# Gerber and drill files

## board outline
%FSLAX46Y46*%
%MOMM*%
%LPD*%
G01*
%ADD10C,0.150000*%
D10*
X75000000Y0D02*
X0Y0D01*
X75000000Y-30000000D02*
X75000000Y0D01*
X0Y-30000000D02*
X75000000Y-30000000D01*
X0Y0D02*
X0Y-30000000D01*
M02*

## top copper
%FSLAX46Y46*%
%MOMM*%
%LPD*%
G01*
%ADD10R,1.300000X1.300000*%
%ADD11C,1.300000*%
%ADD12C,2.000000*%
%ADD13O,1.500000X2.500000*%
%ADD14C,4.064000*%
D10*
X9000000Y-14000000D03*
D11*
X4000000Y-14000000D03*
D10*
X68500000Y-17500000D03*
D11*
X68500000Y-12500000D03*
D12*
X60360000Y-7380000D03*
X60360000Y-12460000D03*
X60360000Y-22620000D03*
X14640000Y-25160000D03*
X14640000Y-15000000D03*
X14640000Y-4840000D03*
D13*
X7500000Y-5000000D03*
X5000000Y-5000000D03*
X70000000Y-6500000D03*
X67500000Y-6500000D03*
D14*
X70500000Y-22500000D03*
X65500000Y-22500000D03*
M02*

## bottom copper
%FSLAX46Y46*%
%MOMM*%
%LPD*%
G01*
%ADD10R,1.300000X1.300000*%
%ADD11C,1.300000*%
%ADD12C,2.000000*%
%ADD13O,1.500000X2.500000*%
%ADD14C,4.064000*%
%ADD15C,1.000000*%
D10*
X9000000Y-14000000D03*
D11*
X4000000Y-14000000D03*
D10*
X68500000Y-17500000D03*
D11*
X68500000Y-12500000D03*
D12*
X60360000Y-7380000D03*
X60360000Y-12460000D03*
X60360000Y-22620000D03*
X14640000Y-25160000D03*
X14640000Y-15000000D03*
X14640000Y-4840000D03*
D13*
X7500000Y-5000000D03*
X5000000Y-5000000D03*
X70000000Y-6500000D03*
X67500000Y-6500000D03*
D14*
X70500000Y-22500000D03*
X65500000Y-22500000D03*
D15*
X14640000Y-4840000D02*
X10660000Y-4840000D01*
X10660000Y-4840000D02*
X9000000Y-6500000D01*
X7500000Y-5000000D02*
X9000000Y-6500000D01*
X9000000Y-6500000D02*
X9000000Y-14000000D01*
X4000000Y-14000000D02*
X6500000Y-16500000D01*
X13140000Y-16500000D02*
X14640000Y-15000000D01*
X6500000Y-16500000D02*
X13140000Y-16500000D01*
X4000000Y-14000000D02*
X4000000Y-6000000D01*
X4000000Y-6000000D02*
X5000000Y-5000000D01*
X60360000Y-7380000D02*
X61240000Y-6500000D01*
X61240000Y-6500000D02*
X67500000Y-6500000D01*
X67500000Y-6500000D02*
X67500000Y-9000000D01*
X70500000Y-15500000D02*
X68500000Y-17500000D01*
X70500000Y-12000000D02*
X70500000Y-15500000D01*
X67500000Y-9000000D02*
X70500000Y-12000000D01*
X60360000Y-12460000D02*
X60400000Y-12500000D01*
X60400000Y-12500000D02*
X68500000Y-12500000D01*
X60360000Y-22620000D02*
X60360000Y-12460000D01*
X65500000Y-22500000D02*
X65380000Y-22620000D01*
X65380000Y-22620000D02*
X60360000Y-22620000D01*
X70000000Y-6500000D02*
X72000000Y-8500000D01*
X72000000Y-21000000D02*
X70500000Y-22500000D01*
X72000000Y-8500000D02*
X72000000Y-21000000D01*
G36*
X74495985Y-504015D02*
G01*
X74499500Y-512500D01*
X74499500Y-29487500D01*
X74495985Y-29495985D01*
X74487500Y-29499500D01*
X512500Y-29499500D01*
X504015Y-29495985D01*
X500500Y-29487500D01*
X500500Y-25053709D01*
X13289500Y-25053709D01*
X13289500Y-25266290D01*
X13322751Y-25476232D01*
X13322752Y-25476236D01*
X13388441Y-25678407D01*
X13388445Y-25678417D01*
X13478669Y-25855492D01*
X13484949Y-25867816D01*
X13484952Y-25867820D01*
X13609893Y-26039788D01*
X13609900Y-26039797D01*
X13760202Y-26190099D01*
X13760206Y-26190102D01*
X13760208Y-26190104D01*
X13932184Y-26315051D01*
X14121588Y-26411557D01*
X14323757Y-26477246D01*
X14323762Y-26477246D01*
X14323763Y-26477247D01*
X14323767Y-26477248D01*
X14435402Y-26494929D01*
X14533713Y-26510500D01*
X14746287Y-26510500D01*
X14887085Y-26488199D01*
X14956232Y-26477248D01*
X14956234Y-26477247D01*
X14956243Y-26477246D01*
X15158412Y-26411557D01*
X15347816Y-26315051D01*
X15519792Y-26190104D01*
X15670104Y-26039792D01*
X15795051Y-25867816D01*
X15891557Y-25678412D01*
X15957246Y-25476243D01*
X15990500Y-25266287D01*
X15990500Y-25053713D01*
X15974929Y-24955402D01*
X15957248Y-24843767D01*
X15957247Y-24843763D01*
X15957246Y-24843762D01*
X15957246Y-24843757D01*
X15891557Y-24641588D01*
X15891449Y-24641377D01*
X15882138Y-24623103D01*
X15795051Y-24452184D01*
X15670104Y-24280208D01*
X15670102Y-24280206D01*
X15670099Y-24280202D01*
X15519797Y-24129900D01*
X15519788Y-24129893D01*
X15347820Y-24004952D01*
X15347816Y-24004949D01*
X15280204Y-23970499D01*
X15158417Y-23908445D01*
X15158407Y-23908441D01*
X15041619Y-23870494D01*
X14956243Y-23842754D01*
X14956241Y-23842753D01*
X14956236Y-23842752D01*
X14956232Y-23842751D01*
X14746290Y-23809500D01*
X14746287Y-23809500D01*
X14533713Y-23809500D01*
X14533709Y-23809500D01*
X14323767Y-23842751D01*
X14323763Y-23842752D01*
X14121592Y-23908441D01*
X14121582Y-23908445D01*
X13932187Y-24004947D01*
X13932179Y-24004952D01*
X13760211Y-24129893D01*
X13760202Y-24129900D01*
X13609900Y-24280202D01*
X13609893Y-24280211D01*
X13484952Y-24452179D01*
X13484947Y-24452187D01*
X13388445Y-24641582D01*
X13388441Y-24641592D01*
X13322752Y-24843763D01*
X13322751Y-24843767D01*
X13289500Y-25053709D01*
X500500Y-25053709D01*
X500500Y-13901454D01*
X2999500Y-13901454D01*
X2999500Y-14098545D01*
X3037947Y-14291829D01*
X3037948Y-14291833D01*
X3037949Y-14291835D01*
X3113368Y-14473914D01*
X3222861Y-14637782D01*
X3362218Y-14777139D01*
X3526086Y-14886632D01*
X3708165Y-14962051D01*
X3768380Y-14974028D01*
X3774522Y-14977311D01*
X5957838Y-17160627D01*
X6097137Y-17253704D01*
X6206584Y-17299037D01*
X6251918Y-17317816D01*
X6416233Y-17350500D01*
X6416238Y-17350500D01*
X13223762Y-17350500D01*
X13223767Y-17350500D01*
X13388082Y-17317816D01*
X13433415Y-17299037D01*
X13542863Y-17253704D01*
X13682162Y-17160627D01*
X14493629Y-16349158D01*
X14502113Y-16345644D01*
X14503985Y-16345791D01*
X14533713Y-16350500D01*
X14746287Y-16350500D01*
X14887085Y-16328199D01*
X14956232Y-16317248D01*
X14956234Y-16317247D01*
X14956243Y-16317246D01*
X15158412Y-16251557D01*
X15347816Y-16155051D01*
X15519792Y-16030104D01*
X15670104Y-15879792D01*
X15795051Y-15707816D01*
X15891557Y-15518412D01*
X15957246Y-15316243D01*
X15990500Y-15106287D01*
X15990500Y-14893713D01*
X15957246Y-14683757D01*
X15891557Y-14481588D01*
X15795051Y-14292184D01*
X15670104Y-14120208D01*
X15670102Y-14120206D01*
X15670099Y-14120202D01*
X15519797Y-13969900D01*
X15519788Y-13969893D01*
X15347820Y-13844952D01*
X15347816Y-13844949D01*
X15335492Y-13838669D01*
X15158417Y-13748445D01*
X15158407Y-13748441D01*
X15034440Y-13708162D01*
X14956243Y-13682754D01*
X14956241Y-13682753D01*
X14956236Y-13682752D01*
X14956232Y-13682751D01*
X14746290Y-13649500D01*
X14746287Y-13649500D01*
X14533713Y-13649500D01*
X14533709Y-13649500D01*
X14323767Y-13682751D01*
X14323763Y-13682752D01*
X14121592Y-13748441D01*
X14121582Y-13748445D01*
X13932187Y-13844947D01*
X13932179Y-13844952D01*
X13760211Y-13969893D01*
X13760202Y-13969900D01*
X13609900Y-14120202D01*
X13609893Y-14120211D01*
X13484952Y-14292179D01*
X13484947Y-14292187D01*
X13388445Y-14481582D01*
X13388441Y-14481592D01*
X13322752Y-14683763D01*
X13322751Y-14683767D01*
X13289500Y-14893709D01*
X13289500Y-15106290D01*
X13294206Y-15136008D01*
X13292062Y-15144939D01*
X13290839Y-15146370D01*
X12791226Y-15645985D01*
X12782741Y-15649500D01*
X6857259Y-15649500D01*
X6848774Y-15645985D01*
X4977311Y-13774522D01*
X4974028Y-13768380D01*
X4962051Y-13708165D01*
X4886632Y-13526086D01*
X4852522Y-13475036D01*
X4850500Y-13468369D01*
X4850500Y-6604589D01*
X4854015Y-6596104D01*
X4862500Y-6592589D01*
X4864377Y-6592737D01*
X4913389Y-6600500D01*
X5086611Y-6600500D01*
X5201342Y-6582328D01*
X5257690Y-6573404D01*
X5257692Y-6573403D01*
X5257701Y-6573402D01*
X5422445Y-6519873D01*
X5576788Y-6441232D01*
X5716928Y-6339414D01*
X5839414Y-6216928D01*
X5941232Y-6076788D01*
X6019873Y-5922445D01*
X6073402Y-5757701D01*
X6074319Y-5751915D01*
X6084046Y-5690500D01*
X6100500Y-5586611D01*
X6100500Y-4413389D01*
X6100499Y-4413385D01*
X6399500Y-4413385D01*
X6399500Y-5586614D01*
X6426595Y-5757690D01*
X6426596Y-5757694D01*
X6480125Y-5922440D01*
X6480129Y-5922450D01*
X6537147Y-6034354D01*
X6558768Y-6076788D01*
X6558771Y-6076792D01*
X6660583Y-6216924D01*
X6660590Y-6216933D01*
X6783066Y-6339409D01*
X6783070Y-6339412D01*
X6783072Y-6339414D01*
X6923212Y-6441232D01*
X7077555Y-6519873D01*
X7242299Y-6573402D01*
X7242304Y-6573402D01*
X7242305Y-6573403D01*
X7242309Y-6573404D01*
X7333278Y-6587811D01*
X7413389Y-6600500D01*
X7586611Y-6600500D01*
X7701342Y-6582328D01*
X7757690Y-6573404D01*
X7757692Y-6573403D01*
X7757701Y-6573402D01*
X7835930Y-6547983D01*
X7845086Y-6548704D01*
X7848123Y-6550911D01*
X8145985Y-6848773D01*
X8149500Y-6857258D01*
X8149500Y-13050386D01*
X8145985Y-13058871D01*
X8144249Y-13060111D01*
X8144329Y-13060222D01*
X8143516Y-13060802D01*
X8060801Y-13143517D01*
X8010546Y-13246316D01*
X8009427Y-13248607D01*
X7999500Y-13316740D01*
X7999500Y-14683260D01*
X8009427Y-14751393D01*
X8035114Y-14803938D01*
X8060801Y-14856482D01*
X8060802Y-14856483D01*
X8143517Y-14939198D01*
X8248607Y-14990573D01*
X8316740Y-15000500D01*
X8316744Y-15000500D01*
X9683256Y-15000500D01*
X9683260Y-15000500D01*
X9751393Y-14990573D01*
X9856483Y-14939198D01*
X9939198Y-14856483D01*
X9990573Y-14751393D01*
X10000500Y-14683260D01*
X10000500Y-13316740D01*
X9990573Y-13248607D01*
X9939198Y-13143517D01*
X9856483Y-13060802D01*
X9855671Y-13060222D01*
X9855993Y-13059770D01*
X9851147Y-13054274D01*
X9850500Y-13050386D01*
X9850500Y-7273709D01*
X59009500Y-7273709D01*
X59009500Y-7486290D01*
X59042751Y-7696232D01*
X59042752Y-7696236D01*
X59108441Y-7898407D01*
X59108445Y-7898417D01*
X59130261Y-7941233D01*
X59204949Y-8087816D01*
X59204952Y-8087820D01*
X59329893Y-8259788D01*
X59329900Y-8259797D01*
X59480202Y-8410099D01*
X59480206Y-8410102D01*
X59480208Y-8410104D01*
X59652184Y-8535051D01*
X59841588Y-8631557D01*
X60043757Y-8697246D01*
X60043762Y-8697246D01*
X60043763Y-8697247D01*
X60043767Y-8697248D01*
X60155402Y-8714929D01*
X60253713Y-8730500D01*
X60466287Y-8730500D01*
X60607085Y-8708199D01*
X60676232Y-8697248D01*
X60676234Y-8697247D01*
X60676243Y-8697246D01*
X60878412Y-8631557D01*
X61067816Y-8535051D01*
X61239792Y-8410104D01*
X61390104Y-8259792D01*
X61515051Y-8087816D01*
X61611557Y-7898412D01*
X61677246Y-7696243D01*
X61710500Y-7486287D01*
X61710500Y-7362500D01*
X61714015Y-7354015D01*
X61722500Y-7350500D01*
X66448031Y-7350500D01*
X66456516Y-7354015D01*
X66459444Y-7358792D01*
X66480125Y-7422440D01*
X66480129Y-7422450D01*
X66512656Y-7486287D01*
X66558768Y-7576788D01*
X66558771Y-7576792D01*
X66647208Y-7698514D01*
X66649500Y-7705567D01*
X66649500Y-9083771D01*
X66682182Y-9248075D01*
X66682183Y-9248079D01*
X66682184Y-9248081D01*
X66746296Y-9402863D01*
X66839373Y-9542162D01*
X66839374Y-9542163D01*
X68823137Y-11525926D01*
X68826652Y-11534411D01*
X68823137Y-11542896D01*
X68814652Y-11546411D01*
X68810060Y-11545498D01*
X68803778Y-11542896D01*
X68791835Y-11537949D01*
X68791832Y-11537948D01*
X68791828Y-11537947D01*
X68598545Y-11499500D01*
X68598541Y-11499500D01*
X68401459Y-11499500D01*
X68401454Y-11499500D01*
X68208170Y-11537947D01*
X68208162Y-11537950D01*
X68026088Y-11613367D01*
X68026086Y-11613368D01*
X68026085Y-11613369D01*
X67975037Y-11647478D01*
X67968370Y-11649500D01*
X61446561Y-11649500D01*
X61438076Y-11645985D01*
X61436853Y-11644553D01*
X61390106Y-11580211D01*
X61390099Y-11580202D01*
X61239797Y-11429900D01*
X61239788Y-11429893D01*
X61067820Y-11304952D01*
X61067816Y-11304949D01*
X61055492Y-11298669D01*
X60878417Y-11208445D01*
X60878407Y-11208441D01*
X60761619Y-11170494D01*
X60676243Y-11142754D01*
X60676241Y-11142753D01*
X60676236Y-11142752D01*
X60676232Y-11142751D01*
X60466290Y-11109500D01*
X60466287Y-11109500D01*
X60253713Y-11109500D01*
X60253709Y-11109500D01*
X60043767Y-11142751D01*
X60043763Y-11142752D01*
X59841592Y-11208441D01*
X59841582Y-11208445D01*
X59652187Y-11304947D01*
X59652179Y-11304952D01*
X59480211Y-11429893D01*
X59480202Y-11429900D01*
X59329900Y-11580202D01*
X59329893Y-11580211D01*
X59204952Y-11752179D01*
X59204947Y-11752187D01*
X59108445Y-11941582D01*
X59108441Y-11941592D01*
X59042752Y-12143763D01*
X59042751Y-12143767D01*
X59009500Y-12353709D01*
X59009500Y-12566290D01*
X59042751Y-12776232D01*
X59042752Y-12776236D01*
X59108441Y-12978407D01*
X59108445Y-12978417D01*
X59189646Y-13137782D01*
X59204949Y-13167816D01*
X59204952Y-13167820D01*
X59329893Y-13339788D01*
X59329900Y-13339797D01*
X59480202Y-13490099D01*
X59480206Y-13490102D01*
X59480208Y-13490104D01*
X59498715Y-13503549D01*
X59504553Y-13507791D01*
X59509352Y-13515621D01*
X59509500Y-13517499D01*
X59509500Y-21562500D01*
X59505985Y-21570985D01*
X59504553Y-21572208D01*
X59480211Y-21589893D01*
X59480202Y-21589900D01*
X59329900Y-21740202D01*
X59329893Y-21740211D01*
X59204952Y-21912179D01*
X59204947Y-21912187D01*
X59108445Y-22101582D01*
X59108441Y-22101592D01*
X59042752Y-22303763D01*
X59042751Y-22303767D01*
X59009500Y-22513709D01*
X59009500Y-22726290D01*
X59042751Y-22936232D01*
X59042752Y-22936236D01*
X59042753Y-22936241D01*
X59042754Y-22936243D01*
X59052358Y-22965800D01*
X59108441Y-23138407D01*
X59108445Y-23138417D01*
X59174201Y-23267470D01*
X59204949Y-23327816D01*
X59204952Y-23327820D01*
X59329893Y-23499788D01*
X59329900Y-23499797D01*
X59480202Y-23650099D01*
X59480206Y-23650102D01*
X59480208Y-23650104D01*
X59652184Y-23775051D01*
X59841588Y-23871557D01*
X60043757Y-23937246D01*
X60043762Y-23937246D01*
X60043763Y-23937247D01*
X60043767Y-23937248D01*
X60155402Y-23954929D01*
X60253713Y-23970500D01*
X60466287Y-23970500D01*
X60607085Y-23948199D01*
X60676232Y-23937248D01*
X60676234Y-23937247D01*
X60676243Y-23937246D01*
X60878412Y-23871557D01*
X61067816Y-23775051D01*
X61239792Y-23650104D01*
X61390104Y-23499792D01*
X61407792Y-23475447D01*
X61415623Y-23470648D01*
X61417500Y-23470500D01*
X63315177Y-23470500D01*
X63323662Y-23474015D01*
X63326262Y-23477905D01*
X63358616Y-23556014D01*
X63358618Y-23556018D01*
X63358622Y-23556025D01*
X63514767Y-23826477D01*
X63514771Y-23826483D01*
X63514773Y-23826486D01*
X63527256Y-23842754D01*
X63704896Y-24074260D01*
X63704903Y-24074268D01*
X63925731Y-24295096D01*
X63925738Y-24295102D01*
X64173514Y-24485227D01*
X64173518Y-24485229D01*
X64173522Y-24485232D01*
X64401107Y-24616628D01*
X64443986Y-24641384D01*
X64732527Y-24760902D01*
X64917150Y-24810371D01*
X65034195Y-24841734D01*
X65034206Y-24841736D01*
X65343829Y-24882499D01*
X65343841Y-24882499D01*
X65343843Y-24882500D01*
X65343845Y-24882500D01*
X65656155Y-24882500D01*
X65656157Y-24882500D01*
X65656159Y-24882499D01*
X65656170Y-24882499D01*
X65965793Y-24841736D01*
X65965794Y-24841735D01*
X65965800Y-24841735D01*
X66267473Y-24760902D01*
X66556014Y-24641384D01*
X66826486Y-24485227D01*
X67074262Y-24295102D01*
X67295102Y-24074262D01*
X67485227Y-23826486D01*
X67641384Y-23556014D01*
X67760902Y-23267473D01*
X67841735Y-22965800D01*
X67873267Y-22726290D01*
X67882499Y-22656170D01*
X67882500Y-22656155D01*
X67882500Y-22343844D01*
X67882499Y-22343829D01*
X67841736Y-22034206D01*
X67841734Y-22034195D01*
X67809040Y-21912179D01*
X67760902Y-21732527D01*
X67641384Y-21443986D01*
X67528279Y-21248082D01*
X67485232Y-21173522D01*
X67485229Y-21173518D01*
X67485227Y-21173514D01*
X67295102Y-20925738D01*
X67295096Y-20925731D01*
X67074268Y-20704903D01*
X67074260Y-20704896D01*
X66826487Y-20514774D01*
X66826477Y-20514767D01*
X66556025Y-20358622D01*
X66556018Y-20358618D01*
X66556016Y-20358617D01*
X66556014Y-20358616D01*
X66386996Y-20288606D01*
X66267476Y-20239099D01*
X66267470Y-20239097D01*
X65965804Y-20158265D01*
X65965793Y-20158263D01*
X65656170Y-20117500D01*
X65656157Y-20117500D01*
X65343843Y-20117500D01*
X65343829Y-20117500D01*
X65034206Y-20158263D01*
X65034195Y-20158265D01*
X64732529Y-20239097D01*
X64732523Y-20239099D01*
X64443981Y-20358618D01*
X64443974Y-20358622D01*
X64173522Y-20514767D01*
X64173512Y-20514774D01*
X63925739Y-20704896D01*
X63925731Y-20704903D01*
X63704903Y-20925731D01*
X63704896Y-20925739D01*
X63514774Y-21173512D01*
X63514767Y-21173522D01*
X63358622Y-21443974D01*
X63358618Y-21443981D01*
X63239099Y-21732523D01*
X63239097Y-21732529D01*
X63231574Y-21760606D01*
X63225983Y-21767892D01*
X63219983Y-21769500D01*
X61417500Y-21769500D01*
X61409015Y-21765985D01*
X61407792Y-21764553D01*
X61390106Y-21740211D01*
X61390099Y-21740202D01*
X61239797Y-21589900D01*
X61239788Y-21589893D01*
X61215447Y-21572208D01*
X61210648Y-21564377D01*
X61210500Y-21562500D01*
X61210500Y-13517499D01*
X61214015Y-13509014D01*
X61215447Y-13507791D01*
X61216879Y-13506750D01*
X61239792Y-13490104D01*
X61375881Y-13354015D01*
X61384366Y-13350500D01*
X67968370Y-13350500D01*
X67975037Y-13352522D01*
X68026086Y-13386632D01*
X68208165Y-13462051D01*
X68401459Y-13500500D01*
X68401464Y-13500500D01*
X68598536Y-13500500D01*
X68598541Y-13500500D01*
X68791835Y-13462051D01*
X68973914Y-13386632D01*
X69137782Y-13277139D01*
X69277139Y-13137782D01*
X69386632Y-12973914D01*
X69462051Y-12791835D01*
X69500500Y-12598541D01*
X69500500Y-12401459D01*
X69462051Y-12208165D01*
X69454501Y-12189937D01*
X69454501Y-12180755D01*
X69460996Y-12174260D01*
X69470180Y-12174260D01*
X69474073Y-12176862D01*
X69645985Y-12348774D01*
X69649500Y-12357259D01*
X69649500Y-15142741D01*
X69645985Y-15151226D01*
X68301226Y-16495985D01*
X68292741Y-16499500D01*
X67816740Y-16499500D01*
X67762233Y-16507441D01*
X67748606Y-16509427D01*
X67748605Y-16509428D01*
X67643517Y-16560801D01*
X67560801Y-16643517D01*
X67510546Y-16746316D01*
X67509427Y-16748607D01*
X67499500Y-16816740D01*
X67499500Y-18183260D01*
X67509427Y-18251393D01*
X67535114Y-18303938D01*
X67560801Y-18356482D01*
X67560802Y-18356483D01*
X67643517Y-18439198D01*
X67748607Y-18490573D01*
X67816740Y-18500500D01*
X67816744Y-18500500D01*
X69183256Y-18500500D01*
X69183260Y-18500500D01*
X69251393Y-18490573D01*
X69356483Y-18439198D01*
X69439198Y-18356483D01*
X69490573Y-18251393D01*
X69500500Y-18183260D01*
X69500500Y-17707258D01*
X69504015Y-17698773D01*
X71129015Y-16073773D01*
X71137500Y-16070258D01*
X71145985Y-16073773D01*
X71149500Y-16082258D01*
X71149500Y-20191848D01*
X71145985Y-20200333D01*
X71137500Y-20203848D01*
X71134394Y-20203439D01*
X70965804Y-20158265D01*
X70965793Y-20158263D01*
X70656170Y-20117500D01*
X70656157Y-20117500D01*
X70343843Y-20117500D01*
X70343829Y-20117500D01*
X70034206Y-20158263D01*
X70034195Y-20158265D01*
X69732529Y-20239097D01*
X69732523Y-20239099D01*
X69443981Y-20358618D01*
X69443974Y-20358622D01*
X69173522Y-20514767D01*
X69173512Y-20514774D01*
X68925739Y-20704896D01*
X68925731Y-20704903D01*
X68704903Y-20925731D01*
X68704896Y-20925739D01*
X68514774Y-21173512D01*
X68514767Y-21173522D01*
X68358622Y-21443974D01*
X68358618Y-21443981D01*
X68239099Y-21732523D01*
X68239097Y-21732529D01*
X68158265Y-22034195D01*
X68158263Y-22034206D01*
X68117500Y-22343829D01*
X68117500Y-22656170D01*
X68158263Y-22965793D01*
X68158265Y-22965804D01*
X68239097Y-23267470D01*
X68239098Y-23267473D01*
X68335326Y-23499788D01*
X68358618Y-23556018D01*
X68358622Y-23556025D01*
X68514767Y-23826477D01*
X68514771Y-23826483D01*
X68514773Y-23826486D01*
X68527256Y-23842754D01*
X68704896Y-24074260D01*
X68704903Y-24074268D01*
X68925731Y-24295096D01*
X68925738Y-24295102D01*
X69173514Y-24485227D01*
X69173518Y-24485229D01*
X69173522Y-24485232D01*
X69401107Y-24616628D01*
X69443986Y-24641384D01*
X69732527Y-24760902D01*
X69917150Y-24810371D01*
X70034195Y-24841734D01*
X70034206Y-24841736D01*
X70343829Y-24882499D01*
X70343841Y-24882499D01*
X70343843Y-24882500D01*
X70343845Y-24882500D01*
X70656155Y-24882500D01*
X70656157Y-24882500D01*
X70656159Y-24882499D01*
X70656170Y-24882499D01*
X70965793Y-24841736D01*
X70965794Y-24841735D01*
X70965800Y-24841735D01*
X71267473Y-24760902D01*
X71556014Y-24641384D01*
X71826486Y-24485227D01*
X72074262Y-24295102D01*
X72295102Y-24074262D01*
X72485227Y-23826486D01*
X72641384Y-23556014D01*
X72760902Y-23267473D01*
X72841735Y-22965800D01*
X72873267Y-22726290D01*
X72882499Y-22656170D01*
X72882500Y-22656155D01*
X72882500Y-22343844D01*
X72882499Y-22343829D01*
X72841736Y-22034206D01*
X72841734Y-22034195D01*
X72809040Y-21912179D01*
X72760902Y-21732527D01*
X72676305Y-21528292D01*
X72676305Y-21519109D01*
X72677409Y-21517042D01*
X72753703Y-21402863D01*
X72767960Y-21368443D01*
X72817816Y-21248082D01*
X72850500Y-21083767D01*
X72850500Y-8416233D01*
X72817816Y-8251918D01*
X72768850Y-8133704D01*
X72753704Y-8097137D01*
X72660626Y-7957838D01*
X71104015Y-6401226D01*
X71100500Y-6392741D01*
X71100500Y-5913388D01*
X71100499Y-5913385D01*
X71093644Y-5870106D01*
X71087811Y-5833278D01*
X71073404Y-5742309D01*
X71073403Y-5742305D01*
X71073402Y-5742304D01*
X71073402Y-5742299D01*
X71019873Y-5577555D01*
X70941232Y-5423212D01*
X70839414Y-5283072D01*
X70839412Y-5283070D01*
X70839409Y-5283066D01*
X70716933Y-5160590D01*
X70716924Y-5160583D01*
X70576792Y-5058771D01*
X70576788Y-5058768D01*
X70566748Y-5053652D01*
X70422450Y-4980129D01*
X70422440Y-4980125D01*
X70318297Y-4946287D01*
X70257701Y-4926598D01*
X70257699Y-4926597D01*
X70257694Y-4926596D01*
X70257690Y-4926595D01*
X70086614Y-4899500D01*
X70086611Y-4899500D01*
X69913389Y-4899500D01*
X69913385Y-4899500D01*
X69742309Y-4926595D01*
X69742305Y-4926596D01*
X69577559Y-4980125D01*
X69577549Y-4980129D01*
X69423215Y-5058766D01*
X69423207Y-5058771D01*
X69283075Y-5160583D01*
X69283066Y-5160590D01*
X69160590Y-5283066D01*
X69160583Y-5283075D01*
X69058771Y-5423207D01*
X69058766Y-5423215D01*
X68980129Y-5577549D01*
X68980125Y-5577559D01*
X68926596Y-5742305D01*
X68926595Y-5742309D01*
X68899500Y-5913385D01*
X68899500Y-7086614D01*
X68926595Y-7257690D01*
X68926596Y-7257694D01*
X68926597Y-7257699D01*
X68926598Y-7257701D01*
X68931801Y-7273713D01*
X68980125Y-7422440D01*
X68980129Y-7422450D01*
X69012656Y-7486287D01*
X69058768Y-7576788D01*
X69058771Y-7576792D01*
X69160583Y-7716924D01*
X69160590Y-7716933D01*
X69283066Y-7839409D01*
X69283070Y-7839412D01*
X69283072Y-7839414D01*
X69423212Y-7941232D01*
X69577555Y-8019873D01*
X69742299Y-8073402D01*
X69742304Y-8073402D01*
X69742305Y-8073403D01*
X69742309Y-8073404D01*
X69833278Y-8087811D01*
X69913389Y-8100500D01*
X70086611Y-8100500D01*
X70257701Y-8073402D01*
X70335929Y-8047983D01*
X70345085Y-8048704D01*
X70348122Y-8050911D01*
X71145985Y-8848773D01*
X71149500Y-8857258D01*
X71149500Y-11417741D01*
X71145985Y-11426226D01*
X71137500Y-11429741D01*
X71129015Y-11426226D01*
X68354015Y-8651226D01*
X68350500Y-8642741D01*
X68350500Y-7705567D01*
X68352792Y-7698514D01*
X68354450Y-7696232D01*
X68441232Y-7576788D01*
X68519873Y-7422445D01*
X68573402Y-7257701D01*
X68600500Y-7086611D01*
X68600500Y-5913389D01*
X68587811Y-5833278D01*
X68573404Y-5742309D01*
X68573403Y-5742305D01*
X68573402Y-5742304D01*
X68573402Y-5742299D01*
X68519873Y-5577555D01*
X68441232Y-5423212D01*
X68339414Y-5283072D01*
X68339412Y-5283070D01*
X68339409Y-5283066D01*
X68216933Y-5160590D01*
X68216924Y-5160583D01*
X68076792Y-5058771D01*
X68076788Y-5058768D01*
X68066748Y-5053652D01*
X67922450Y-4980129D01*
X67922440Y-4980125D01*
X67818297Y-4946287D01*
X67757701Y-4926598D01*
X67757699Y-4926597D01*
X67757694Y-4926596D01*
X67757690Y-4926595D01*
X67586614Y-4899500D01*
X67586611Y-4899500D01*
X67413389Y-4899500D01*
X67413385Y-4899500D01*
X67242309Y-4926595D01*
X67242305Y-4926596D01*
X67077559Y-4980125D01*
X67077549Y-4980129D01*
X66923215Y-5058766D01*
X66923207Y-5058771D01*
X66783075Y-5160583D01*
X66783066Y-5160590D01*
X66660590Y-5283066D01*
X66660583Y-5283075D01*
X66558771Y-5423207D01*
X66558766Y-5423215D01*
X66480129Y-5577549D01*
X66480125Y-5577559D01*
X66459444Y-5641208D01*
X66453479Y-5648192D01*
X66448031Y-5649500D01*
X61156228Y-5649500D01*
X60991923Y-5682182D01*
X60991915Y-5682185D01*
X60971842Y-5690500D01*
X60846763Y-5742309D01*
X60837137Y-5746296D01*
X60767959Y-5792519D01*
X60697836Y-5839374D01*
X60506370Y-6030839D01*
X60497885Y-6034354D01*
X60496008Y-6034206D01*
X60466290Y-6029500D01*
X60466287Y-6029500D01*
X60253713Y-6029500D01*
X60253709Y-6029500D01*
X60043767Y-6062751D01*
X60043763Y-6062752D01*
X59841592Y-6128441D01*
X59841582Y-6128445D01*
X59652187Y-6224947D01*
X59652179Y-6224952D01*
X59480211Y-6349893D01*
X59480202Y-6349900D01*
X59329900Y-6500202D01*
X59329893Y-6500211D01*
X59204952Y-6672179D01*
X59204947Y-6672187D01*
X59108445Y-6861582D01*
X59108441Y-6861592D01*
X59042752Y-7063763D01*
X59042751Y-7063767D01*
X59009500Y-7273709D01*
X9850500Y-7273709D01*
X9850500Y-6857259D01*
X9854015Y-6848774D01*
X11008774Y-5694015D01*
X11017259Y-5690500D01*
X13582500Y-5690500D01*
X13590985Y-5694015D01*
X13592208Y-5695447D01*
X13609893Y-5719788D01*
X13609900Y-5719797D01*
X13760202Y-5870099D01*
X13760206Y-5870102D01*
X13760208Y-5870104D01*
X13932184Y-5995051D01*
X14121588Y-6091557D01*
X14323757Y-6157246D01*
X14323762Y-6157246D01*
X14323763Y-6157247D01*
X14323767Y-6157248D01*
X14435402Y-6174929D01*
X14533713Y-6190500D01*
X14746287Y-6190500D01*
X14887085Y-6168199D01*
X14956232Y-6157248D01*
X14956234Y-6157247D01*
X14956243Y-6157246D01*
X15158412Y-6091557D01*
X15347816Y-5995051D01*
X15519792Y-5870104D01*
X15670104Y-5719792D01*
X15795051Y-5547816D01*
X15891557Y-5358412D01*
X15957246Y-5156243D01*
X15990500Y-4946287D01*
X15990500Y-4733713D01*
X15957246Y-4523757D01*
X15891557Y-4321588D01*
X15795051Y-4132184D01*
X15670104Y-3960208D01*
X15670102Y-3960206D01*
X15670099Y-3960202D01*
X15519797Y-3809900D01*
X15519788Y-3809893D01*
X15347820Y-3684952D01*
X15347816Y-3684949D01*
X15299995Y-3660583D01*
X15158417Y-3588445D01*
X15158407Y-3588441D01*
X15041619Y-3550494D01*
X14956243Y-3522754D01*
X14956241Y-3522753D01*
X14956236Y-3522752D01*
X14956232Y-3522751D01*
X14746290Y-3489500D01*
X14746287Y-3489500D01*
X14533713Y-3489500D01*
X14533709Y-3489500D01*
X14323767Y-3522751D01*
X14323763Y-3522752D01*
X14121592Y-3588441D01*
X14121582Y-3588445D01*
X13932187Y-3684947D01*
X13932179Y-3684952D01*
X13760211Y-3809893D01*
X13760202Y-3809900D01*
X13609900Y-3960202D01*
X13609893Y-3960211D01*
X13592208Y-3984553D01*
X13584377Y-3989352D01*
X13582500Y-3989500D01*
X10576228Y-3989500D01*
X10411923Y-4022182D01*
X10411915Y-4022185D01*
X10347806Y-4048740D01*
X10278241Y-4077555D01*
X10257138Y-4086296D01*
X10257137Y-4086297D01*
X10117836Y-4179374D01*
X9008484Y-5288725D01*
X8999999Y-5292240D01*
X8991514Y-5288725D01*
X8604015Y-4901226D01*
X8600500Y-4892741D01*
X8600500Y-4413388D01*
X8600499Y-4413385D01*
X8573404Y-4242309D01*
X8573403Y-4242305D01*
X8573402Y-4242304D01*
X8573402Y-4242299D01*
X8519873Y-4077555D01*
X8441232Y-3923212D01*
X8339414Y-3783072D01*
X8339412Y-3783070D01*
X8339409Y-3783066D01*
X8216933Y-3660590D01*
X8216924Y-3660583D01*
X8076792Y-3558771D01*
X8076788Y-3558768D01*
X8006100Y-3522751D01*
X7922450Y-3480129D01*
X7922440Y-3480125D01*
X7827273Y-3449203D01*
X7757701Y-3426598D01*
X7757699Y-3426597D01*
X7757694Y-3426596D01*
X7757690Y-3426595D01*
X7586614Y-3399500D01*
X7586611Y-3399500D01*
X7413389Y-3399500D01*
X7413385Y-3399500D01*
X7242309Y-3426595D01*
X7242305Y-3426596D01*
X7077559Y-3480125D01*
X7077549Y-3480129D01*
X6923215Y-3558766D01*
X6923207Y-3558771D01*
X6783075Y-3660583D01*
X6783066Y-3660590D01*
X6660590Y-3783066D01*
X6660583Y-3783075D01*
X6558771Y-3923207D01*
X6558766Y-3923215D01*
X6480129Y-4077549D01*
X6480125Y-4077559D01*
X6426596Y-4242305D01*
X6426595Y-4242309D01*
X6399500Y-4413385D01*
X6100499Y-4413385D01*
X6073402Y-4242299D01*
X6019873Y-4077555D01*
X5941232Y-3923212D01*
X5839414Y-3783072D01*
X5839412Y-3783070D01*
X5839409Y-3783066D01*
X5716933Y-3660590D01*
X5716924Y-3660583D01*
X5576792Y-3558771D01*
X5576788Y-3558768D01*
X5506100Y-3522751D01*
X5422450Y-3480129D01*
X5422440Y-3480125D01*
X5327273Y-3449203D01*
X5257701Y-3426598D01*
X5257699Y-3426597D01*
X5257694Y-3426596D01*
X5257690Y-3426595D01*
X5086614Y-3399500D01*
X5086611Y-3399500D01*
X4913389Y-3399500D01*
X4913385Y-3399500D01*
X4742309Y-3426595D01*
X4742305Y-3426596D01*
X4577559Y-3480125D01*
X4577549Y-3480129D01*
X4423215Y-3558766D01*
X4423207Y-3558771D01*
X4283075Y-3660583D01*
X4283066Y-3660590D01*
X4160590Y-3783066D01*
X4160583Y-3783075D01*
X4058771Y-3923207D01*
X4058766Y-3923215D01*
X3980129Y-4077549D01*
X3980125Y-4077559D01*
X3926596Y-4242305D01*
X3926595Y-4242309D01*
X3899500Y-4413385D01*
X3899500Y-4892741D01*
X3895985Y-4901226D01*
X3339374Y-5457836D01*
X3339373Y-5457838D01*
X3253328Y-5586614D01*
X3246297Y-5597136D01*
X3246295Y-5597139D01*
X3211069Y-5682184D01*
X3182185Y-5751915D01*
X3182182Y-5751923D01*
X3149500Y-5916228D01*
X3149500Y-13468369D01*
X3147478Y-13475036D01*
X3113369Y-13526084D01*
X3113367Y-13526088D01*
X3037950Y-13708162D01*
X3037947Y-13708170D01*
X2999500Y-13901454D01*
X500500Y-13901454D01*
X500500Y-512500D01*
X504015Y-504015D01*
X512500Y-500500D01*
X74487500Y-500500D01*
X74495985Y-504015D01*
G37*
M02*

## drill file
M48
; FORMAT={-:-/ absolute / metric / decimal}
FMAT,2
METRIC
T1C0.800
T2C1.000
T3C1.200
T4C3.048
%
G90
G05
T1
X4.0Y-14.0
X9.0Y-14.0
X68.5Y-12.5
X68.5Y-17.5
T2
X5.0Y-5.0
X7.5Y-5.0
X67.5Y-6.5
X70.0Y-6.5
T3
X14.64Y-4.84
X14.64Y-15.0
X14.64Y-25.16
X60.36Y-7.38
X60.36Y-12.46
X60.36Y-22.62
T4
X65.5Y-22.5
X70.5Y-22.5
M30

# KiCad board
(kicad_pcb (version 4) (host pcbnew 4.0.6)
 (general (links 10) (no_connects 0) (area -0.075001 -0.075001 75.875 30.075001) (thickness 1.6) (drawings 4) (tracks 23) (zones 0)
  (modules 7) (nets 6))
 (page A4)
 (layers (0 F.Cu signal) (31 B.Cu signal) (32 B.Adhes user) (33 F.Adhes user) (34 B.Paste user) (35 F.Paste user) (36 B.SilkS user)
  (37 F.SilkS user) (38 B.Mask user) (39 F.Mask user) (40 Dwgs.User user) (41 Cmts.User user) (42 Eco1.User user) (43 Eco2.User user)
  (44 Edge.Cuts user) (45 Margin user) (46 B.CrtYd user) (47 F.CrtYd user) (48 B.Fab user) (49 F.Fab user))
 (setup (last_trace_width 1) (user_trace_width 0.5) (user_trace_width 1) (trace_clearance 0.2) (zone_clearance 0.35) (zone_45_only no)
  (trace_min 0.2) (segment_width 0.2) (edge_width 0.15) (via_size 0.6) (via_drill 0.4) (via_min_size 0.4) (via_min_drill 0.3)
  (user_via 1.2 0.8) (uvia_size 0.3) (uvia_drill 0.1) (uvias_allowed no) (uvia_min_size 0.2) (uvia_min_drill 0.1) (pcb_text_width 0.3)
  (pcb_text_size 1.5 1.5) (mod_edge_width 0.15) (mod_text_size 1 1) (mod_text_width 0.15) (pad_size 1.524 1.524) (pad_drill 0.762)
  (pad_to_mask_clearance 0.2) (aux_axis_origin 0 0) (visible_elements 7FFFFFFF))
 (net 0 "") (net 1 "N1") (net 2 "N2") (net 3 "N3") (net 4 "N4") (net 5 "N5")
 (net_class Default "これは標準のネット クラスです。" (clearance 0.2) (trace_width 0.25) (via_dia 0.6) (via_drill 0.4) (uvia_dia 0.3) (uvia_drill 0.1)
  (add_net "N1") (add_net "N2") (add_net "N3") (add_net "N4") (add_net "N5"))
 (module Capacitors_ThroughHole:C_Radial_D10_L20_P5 (layer F.Cu) (at 9 14 180)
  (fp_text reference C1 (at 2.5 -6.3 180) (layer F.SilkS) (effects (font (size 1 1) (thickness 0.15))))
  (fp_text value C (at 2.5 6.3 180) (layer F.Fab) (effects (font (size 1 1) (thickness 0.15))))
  (pad 1 thru_hole rect (at 0 0 180) (size 1.3 1.3) (drill 0.8) (layers *.Cu *.Mask F.SilkS) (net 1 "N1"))
  (pad 2 thru_hole circle (at 5 0 180) (size 1.3 1.3) (drill 0.8) (layers *.Cu *.Mask F.SilkS) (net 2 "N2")))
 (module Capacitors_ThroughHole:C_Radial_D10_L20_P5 (layer F.Cu) (at 68.5 17.5 90)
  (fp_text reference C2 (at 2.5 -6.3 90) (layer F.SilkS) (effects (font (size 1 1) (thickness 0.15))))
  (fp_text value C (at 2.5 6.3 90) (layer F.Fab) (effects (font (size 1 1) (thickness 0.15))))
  (pad 1 thru_hole rect (at 0 0 90) (size 1.3 1.3) (drill 0.8) (layers *.Cu *.Mask F.SilkS) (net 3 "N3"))
  (pad 2 thru_hole circle (at 5 0 90) (size 1.3 1.3) (drill 0.8) (layers *.Cu *.Mask F.SilkS) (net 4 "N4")))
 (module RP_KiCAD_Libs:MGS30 (layer F.Cu) (at 37.5 15)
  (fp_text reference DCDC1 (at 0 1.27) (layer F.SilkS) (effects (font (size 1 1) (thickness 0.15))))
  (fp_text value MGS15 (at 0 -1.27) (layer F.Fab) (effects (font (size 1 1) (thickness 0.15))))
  (pad 6 thru_hole circle (at 22.86 -7.62) (size 2 2) (drill 1.2) (layers *.Cu *.Mask) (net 3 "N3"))
  (pad 5 thru_hole circle (at 22.86 -2.54) (size 2 2) (drill 1.2) (layers *.Cu *.Mask) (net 4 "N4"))
  (pad 4 thru_hole circle (at 22.86 7.62) (size 2 2) (drill 1.2) (layers *.Cu *.Mask) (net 4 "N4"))
  (pad 2 thru_hole circle (at -22.86 10.16) (size 2 2) (drill 1.2) (layers *.Cu *.Mask))
  (pad 3 thru_hole circle (at -22.86 0) (size 2 2) (drill 1.2) (layers *.Cu *.Mask) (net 2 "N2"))
  (pad 1 thru_hole circle (at -22.86 -10.16) (size 2 2) (drill 1.2) (layers *.Cu *.Mask) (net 1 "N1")))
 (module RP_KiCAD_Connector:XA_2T (layer F.Cu) (at 7.5 5 180)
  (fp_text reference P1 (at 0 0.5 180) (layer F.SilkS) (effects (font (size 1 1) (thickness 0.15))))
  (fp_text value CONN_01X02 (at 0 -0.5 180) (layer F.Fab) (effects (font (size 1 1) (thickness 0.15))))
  (pad 2 thru_hole oval (at 0 0 180) (size 1.5 2.5) (drill 1) (layers *.Cu *.Mask F.SilkS) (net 1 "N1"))
  (pad 1 thru_hole oval (at 2.5 0 180) (size 1.5 2.5) (drill 1) (layers *.Cu *.Mask F.SilkS) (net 2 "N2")))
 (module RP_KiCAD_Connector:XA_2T (layer F.Cu) (at 70 6.5 180)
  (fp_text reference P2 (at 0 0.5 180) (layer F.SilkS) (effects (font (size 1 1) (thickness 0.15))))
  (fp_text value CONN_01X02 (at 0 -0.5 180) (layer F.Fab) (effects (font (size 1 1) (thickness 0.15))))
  (pad 2 thru_hole oval (at 0 0 180) (size 1.5 2.5) (drill 1) (layers *.Cu *.Mask F.SilkS) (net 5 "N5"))
  (pad 1 thru_hole oval (at 2.5 0 180) (size 1.5 2.5) (drill 1) (layers *.Cu *.Mask F.SilkS) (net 3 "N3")))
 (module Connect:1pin (layer F.Cu) (at 70.5 22.5)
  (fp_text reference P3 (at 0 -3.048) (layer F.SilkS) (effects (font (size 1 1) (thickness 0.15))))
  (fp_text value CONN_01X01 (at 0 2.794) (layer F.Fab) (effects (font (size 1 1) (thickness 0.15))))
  (pad 1 thru_hole circle (at 0 0) (size 4.064 4.064) (drill 3.048) (layers *.Cu *.Mask F.SilkS) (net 5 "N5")))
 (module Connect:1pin (layer F.Cu) (at 65.5 22.5)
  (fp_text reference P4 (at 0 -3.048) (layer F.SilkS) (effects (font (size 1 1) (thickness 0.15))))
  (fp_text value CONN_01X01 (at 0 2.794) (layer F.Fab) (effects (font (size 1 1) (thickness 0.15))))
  (pad 1 thru_hole circle (at 0 0) (size 4.064 4.064) (drill 3.048) (layers *.Cu *.Mask F.SilkS) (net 4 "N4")))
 (gr_line (start 75 0) (end 0 0) (angle 90) (layer Edge.Cuts) (width 0.15))
 (gr_line (start 75 30) (end 75 0) (angle 90) (layer Edge.Cuts) (width 0.15))
 (gr_line (start 0 30) (end 75 30) (angle 90) (layer Edge.Cuts) (width 0.15))
 (gr_line (start 0 0) (end 0 30) (angle 90) (layer Edge.Cuts) (width 0.15))
 (segment (start 14.64 4.84) (end 10.66 4.84) (width 1) (layer B.Cu) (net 1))
 (segment (start 10.66 4.84) (end 9 6.5) (width 1) (layer B.Cu) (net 1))
 (segment (start 7.5 5) (end 9 6.5) (width 1) (layer B.Cu) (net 1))
 (segment (start 9 6.5) (end 9 14) (width 1) (layer B.Cu) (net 1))
 (segment (start 4 14) (end 6.5 16.5) (width 1) (layer B.Cu) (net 2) (status 400000))
 (segment (start 13.14 16.5) (end 14.64 15) (width 1) (layer B.Cu) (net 2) (status 800000))
 (segment (start 6.5 16.5) (end 13.14 16.5) (width 1) (layer B.Cu) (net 2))
 (segment (start 4 14) (end 4 6) (width 1) (layer B.Cu) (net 2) (status 400000))
 (segment (start 4 6) (end 5 5) (width 1) (layer B.Cu) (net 2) (status 800000))
 (segment (start 60.36 7.38) (end 61.24 6.5) (width 1) (layer B.Cu) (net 3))
 (segment (start 61.24 6.5) (end 67.5 6.5) (width 1) (layer B.Cu) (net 3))
 (segment (start 67.5 6.5) (end 67.5 9) (width 1) (layer B.Cu) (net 3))
 (segment (start 70.5 15.5) (end 68.5 17.5) (width 1) (layer B.Cu) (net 3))
 (segment (start 70.5 12) (end 70.5 15.5) (width 1) (layer B.Cu) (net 3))
 (segment (start 67.5 9) (end 70.5 12) (width 1) (layer B.Cu) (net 3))
 (segment (start 60.36 12.46) (end 60.4 12.5) (width 1) (layer B.Cu) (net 4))
 (segment (start 60.4 12.5) (end 68.5 12.5) (width 1) (layer B.Cu) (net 4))
 (segment (start 60.36 22.62) (end 60.36 12.46) (width 1) (layer B.Cu) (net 4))
 (segment (start 65.5 22.5) (end 65.38 22.62) (width 1) (layer B.Cu) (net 4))
 (segment (start 65.38 22.62) (end 60.36 22.62) (width 1) (layer B.Cu) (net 4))
 (segment (start 70 6.5) (end 72 8.5) (width 1) (layer B.Cu) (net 5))
 (segment (start 72 21) (end 70.5 22.5) (width 1) (layer B.Cu) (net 5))
 (segment (start 72 8.5) (end 72 21) (width 1) (layer B.Cu) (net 5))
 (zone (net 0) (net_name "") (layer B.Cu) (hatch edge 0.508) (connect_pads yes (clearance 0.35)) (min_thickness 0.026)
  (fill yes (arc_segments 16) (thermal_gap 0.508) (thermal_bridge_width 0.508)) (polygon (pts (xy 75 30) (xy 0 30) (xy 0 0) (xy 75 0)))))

